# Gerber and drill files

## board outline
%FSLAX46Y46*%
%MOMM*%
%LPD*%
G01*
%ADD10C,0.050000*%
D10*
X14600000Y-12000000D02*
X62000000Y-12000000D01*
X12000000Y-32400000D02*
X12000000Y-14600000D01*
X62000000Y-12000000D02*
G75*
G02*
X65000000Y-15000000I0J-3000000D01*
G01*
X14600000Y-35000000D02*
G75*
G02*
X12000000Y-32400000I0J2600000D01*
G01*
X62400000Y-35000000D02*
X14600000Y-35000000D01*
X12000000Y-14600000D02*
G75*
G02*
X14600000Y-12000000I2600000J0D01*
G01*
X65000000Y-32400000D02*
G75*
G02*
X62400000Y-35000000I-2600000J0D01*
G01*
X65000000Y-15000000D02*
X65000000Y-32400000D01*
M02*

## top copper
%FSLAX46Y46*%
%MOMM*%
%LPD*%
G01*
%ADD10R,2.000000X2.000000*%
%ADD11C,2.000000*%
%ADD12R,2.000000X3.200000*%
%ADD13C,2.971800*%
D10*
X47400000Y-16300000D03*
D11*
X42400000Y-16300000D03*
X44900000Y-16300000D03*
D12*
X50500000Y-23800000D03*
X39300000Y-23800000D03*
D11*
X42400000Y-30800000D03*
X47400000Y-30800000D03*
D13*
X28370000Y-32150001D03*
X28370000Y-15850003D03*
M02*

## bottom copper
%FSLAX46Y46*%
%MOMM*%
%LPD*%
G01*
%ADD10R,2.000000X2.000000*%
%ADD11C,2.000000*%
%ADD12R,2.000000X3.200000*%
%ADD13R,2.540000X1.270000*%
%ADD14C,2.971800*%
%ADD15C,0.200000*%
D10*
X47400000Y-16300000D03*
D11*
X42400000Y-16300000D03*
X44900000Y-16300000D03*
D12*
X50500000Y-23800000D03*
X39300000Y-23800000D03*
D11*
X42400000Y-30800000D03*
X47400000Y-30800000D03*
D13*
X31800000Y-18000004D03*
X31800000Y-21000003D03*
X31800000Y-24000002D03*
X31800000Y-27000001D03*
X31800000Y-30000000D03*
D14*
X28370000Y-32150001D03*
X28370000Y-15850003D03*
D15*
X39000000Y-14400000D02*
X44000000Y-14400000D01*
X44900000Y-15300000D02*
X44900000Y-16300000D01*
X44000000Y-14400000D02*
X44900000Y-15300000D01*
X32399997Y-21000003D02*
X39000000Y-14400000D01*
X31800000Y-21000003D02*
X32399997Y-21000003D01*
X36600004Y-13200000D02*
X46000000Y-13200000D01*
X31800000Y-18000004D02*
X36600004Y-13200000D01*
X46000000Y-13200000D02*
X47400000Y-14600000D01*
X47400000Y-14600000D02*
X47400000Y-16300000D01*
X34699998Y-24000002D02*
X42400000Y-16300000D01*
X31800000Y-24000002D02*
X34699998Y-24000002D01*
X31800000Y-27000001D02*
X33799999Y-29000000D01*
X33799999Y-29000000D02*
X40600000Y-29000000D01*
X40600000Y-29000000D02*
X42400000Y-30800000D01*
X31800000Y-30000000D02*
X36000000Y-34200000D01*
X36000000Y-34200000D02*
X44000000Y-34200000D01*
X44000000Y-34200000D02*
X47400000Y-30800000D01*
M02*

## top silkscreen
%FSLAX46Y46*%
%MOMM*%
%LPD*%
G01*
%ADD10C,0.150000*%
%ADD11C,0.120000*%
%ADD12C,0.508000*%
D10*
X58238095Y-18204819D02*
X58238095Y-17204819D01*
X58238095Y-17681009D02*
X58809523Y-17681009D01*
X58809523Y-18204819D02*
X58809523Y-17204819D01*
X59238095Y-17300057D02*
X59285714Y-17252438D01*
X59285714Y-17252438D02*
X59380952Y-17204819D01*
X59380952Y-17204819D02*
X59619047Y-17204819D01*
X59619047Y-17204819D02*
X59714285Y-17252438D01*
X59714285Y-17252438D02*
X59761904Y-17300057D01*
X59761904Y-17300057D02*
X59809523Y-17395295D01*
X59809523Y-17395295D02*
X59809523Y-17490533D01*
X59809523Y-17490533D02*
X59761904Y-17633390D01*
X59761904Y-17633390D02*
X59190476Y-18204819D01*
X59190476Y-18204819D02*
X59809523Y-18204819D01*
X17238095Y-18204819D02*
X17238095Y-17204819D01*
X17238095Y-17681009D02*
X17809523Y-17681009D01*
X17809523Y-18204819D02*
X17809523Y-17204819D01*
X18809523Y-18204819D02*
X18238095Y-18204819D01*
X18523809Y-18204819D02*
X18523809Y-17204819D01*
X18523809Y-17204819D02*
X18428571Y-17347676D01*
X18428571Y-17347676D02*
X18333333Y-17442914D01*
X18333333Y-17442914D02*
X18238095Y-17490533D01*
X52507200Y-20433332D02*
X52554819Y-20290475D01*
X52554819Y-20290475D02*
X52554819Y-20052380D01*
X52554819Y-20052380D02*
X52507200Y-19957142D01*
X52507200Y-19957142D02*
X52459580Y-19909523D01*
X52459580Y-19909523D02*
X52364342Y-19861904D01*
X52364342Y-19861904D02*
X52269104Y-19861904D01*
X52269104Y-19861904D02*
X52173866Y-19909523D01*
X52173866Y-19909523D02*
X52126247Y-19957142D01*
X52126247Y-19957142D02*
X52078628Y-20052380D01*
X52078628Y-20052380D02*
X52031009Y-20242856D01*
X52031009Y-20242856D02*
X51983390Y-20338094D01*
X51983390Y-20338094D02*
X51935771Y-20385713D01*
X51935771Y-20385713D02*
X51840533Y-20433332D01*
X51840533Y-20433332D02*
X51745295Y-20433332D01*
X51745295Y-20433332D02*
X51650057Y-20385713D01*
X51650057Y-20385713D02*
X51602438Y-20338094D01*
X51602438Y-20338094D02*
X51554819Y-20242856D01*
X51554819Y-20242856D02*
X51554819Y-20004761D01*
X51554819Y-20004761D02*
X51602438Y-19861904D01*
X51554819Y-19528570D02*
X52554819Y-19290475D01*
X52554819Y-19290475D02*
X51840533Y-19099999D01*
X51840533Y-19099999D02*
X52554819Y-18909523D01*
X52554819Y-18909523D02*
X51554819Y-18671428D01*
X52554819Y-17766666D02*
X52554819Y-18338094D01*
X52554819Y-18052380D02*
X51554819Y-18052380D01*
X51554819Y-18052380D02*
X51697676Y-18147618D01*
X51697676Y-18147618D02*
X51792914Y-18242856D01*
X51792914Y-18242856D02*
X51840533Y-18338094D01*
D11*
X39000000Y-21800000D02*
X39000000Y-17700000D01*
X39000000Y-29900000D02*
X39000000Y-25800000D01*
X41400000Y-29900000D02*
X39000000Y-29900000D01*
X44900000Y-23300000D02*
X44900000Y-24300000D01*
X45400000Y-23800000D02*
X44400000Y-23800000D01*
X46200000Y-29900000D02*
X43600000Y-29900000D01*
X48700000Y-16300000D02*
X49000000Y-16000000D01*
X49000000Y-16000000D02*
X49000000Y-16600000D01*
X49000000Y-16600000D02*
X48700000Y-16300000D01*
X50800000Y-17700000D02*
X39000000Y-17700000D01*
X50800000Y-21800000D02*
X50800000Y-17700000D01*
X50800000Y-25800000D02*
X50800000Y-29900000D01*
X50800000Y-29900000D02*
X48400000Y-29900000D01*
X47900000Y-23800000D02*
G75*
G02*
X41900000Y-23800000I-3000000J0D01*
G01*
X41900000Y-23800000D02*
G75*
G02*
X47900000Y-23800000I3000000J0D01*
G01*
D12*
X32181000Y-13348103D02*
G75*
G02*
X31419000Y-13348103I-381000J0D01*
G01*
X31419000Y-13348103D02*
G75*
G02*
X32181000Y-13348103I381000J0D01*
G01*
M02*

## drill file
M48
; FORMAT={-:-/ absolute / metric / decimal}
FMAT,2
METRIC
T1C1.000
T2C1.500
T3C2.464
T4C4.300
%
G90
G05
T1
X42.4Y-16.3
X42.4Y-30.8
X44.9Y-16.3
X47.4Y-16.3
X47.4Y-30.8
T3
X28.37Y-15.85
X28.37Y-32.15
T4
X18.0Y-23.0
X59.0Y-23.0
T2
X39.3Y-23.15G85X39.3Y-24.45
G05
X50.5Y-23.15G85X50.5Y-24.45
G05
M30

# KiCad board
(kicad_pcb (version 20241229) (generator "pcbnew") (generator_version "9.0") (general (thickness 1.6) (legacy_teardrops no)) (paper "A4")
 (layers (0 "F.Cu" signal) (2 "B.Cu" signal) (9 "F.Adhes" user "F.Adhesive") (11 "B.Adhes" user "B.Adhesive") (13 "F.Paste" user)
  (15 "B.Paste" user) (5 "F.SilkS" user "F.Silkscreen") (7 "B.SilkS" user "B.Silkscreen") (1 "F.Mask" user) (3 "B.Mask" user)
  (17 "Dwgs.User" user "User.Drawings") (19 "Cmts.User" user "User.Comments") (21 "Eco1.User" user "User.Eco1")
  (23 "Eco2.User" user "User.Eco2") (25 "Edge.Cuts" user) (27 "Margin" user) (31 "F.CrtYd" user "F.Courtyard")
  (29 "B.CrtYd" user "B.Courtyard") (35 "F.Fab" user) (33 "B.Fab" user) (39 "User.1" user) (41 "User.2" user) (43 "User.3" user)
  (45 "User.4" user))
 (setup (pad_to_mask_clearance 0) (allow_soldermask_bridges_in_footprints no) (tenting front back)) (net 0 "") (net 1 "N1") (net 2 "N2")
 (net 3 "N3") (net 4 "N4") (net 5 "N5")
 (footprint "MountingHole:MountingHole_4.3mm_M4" (layer "F.Cu") (at 59 23)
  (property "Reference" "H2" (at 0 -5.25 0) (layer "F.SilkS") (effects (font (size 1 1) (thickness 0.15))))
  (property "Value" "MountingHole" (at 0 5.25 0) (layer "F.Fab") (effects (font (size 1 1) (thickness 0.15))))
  (pad "" np_thru_hole circle (at 0 0) (size 4.3 4.3) (drill 4.3) (layers "*.Cu" "*.Mask")))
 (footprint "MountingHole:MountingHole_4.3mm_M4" (layer "F.Cu") (at 18 23)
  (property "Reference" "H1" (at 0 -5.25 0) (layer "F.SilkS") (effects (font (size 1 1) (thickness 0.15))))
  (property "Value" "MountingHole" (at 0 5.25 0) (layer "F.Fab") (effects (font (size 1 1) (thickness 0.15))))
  (pad "" np_thru_hole circle (at 0 0) (size 4.3 4.3) (drill 4.3) (layers "*.Cu" "*.Mask")))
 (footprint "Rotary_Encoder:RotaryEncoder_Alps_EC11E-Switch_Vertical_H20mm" (layer "F.Cu") (at 47.4 16.3 -90)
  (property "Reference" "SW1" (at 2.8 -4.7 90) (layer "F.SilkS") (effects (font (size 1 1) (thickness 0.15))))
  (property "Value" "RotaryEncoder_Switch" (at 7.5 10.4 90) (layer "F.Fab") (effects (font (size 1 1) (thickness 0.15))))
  (fp_line (start 5.5 8.4) (end 1.4 8.4) (stroke (width 0.12) (type solid)) (layer "F.SilkS"))
  (fp_line (start 13.6 8.4) (end 9.5 8.4) (stroke (width 0.12) (type solid)) (layer "F.SilkS"))
  (fp_line (start 13.6 6) (end 13.6 8.4) (stroke (width 0.12) (type solid)) (layer "F.SilkS"))
  (fp_line (start 7 2.5) (end 8 2.5) (stroke (width 0.12) (type solid)) (layer "F.SilkS"))
  (fp_line (start 7.5 2) (end 7.5 3) (stroke (width 0.12) (type solid)) (layer "F.SilkS"))
  (fp_line (start 13.6 1.2) (end 13.6 3.8) (stroke (width 0.12) (type solid)) (layer "F.SilkS"))
  (fp_line (start 0 -1.3) (end -0.3 -1.6) (stroke (width 0.12) (type solid)) (layer "F.SilkS"))
  (fp_line (start -0.3 -1.6) (end 0.3 -1.6) (stroke (width 0.12) (type solid)) (layer "F.SilkS"))
  (fp_line (start 0.3 -1.6) (end 0 -1.3) (stroke (width 0.12) (type solid)) (layer "F.SilkS"))
  (fp_line (start 1.4 -3.4) (end 1.4 8.4) (stroke (width 0.12) (type solid)) (layer "F.SilkS"))
  (fp_line (start 5.5 -3.4) (end 1.4 -3.4) (stroke (width 0.12) (type solid)) (layer "F.SilkS"))
  (fp_line (start 9.5 -3.4) (end 13.6 -3.4) (stroke (width 0.12) (type solid)) (layer "F.SilkS"))
  (fp_line (start 13.6 -3.4) (end 13.6 -1) (stroke (width 0.12) (type solid)) (layer "F.SilkS"))
  (fp_circle (center 7.5 2.5) (end 10.5 2.5) (stroke (width 0.12) (type solid)) (fill no) (layer "F.SilkS"))
  (pad "A" thru_hole rect (at 0 0 270) (size 2 2) (drill 1) (layers "*.Cu" "*.Mask") (remove_unused_layers no) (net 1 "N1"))
  (pad "B" thru_hole circle (at 0 5 270) (size 2 2) (drill 1) (layers "*.Cu" "*.Mask") (remove_unused_layers no) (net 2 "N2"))
  (pad "C" thru_hole circle (at 0 2.5 270) (size 2 2) (drill 1) (layers "*.Cu" "*.Mask") (remove_unused_layers no) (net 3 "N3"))
  (pad "MP" thru_hole rect (at 7.5 -3.1 270) (size 3.2 2) (drill oval 2.8 1.5) (layers "*.Cu" "*.Mask") (remove_unused_layers no))
  (pad "MP" thru_hole rect (at 7.5 8.1 270) (size 3.2 2) (drill oval 2.8 1.5) (layers "*.Cu" "*.Mask") (remove_unused_layers no))
  (pad "S1" thru_hole circle (at 14.5 5 270) (size 2 2) (drill 1) (layers "*.Cu" "*.Mask") (remove_unused_layers no) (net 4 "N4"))
  (pad "S2" thru_hole circle (at 14.5 0 270) (size 2 2) (drill 1) (layers "*.Cu" "*.Mask") (remove_unused_layers no) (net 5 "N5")))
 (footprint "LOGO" (layer "B.Cu") (at 44.6 23.8 180)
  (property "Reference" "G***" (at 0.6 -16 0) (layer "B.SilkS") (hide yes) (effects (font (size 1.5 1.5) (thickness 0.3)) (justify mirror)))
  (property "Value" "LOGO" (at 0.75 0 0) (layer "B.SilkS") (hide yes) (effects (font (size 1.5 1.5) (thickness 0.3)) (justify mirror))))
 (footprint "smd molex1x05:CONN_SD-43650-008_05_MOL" (layer "B.Cu") (at 28.688701 24.000002 90)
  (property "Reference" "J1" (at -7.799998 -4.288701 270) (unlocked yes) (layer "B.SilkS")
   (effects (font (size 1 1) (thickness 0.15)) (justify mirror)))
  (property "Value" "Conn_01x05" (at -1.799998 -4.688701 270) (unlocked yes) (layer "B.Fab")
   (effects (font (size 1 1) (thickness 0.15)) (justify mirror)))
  (fp_circle (center 10.651899 3.111299) (end 11.032899 3.111299) (stroke (width 0.508) (type solid)) (fill no) (layer "F.SilkS"))
  (pad "1" smd rect (at 5.999998 3.111299 90) (size 1.27 2.54) (layers "B.Cu" "B.Mask" "B.Paste") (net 1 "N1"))
  (pad "2" smd rect (at 2.999999 3.111299 90) (size 1.27 2.54) (layers "B.Cu" "B.Mask" "B.Paste") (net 3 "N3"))
  (pad "3" smd rect (at 0 3.111299 90) (size 1.27 2.54) (layers "B.Cu" "B.Mask" "B.Paste") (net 2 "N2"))
  (pad "4" smd rect (at -2.999999 3.111299 90) (size 1.27 2.54) (layers "B.Cu" "B.Mask" "B.Paste") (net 4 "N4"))
  (pad "5" smd rect (at -5.999998 3.111299 90) (size 1.27 2.54) (layers "B.Cu" "B.Mask" "B.Paste") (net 5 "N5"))
  (pad "6" thru_hole circle (at -8.149999 -0.318701 90) (size 2.9718 2.9718) (drill 2.4638) (layers "*.Cu" "*.Mask")
   (remove_unused_layers no))
  (pad "7" thru_hole circle (at 8.149999 -0.318701 90) (size 2.9718 2.9718) (drill 2.4638) (layers "*.Cu" "*.Mask")
   (remove_unused_layers no)))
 (gr_line (start 14.6 12) (end 62 12) (stroke (width 0.05) (type default)) (layer "Edge.Cuts"))
 (gr_line (start 12 32.4) (end 12 14.6) (stroke (width 0.05) (type default)) (layer "Edge.Cuts"))
 (gr_arc (start 62 12) (mid 64.12132 12.87868) (end 65 15) (stroke (width 0.05) (type default)) (layer "Edge.Cuts"))
 (gr_arc (start 14.6 35) (mid 12.761522 34.238478) (end 12 32.4) (stroke (width 0.05) (type default)) (layer "Edge.Cuts"))
 (gr_line (start 62.4 35) (end 14.6 35) (stroke (width 0.05) (type default)) (layer "Edge.Cuts"))
 (gr_arc (start 12 14.6) (mid 12.761522 12.761522) (end 14.6 12) (stroke (width 0.05) (type default)) (layer "Edge.Cuts"))
 (gr_arc (start 65 32.4) (mid 64.238478 34.238478) (end 62.4 35) (stroke (width 0.05) (type default)) (layer "Edge.Cuts"))
 (gr_line (start 65 15) (end 65 32.4) (stroke (width 0.05) (type default)) (layer "Edge.Cuts"))
 (segment (start 39 14.4) (end 44 14.4) (width 0.2) (layer "B.Cu") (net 3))
 (segment (start 44.9 15.3) (end 44.9 16.3) (width 0.2) (layer "B.Cu") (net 3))
 (segment (start 44 14.4) (end 44.9 15.3) (width 0.2) (layer "B.Cu") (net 3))
 (segment (start 32.399997 21.000003) (end 39 14.4) (width 0.2) (layer "B.Cu") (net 3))
 (segment (start 31.8 21.000003) (end 32.399997 21.000003) (width 0.2) (layer "B.Cu") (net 3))
 (segment (start 36.600004 13.2) (end 46 13.2) (width 0.2) (layer "B.Cu") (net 1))
 (segment (start 31.8 18.000004) (end 36.600004 13.2) (width 0.2) (layer "B.Cu") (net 1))
 (segment (start 46 13.2) (end 47.4 14.6) (width 0.2) (layer "B.Cu") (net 1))
 (segment (start 47.4 14.6) (end 47.4 16.3) (width 0.2) (layer "B.Cu") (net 1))
 (segment (start 34.699998 24.000002) (end 42.4 16.3) (width 0.2) (layer "B.Cu") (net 2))
 (segment (start 31.8 24.000002) (end 34.699998 24.000002) (width 0.2) (layer "B.Cu") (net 2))
 (segment (start 31.8 27.000001) (end 33.799999 29) (width 0.2) (layer "B.Cu") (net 4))
 (segment (start 33.799999 29) (end 40.6 29) (width 0.2) (layer "B.Cu") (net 4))
 (segment (start 40.6 29) (end 42.4 30.8) (width 0.2) (layer "B.Cu") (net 4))
 (segment (start 31.8 30) (end 36 34.2) (width 0.2) (layer "B.Cu") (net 5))
 (segment (start 36 34.2) (end 44 34.2) (width 0.2) (layer "B.Cu") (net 5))
 (segment (start 44 34.2) (end 47.4 30.8) (width 0.2) (layer "B.Cu") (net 5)))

